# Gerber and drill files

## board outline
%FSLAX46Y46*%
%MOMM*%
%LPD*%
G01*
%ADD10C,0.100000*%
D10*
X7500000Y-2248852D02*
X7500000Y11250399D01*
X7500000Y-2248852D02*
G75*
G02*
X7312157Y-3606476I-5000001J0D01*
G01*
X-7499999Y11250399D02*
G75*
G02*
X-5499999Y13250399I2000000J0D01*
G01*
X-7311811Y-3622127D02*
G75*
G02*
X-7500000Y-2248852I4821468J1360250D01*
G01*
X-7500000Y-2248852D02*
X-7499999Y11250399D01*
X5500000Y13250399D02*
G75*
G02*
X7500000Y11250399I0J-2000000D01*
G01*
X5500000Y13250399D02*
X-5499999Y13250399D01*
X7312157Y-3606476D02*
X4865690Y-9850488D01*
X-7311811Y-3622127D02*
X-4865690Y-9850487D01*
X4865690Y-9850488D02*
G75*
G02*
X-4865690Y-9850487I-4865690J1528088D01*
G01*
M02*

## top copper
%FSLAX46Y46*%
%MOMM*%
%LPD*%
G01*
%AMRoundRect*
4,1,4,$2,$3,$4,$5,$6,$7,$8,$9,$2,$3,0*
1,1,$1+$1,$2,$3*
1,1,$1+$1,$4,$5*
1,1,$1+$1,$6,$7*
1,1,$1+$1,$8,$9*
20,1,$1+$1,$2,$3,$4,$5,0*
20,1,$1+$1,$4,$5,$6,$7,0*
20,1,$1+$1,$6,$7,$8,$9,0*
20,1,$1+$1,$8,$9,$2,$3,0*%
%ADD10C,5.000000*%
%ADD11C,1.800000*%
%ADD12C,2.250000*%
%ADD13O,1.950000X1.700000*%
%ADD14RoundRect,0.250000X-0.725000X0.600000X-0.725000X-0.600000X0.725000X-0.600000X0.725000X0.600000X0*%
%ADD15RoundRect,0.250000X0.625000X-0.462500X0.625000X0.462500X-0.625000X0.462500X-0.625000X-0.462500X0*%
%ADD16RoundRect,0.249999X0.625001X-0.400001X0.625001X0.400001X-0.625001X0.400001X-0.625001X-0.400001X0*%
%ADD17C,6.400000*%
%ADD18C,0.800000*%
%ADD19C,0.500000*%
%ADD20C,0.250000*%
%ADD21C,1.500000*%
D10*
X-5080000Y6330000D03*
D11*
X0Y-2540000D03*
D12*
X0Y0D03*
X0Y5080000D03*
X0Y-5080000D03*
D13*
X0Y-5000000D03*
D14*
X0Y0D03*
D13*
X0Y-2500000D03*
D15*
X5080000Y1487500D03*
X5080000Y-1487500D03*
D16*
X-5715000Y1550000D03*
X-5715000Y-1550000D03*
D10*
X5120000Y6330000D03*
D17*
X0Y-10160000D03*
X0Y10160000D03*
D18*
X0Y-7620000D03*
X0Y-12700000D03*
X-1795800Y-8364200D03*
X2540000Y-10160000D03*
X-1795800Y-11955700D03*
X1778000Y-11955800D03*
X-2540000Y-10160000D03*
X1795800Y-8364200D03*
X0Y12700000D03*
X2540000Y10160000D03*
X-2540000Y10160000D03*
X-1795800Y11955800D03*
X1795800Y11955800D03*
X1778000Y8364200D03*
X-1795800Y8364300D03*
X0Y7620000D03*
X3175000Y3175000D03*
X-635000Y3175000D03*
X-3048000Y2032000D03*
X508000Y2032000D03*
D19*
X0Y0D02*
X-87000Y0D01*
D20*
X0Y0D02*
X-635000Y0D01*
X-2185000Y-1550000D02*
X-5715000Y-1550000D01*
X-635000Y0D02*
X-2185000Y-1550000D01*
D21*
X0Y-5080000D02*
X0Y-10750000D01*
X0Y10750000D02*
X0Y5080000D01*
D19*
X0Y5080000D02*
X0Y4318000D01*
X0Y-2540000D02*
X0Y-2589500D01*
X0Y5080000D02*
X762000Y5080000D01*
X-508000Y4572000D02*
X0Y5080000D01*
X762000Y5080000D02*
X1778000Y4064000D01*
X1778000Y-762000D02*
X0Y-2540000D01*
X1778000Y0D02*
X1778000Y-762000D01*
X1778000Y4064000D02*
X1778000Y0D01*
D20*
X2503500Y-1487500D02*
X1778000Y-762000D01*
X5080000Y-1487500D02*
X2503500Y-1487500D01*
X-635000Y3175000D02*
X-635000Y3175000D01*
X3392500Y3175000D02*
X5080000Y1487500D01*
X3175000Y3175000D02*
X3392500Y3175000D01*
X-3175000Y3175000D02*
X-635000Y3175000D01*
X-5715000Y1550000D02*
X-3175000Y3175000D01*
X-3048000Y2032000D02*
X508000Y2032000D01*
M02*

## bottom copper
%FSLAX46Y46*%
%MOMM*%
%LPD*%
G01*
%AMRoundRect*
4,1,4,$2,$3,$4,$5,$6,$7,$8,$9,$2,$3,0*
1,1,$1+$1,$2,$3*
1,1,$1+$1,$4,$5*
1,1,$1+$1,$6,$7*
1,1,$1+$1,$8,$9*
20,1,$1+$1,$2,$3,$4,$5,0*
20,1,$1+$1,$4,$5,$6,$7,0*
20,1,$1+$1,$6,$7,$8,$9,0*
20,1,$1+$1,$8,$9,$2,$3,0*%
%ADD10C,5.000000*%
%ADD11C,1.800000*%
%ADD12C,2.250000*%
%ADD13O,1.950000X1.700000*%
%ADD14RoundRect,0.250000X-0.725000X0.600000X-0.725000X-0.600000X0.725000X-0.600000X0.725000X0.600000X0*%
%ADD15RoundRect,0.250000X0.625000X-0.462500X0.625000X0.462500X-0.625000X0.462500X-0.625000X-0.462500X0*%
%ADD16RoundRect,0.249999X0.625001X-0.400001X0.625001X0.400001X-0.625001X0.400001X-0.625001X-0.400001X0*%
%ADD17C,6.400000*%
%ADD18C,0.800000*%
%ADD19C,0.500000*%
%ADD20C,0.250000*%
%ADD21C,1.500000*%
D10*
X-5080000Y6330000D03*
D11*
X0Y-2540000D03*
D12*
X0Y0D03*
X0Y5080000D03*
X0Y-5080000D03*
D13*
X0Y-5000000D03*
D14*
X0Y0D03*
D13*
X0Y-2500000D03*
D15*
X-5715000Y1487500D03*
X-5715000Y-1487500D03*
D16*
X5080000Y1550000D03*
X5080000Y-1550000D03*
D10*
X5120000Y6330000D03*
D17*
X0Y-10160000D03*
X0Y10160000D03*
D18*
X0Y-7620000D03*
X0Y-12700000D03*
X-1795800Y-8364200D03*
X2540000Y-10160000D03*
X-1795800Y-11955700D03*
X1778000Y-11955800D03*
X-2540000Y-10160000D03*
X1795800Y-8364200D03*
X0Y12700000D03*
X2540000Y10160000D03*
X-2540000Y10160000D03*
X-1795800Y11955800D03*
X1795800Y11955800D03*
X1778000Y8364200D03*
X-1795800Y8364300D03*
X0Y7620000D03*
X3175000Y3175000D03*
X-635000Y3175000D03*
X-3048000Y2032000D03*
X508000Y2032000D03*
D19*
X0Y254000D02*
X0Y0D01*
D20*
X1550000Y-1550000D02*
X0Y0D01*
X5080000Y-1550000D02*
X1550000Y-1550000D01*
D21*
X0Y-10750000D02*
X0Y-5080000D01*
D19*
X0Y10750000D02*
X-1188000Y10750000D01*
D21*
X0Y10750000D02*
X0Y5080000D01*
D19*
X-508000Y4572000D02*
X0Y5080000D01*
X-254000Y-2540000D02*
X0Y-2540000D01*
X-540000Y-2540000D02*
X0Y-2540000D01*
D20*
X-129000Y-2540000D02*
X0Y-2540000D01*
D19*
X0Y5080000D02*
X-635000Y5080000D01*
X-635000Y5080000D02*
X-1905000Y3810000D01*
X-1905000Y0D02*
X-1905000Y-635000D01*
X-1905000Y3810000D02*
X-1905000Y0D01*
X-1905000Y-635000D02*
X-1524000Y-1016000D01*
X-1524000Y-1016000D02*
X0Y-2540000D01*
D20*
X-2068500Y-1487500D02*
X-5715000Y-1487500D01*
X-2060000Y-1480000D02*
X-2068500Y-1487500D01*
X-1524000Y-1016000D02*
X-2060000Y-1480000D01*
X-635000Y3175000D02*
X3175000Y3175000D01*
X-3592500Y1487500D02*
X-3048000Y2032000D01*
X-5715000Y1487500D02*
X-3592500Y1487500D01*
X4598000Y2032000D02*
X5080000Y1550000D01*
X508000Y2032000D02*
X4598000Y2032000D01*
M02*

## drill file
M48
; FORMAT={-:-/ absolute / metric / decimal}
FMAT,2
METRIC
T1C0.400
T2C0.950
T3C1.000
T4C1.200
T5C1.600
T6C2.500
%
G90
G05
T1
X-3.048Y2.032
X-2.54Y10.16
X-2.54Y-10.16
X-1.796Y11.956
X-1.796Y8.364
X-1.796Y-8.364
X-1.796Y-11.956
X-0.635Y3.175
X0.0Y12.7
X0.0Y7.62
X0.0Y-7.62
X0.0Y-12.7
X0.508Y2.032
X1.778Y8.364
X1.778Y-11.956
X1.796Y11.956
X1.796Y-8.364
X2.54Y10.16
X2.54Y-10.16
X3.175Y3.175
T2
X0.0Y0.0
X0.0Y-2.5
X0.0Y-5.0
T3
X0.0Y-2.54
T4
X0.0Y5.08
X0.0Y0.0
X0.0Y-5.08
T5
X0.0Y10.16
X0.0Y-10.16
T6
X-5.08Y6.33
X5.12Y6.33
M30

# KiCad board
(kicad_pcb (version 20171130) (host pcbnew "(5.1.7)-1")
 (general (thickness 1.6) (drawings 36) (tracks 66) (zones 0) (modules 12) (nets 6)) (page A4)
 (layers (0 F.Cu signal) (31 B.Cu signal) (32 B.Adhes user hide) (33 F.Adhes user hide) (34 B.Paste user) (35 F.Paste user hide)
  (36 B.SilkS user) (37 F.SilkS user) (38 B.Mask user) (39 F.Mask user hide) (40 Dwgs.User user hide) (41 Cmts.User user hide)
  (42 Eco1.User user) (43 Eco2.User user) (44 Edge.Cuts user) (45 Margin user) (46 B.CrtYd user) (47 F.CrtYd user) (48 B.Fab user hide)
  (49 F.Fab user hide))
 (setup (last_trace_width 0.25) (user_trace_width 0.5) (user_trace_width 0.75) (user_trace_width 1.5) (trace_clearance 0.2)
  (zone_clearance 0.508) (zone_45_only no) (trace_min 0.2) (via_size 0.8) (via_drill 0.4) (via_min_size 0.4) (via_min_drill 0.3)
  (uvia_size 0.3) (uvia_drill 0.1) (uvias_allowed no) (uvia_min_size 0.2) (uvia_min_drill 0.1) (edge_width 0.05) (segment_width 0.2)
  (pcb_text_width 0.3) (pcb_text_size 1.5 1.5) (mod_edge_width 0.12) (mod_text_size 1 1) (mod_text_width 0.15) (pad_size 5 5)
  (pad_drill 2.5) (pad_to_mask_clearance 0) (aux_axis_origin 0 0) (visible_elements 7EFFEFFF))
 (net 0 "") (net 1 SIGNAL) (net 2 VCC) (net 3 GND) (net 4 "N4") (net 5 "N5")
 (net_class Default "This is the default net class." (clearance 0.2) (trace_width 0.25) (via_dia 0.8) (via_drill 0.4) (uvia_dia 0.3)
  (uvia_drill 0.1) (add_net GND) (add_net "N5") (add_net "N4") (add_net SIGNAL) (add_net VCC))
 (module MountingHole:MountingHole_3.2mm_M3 (layer F.Cu) (at -5.08 -6.33)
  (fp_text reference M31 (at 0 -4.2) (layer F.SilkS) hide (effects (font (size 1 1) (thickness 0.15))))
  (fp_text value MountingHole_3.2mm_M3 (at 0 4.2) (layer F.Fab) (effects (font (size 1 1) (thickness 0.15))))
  (pad "" np_thru_hole circle (at 0 0) (size 5 5) (drill 2.5) (layers *.Cu *.Mask)))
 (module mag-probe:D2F (layer F.Cu) (at 0 0 270)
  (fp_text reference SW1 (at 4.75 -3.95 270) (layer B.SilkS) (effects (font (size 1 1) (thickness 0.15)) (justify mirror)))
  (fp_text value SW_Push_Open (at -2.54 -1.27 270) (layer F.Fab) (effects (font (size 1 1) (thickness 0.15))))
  (pad 4 thru_hole circle (at 2.54 0 270) (size 1.8 1.8) (drill 1) (layers *.Cu *.Mask) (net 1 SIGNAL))
  (pad 3 thru_hole circle (at 0 0 270) (size 2.25 2.25) (drill 1.2) (layers *.Cu *.Mask) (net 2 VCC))
  (pad 2 thru_hole circle (at -5.08 0 270) (size 2.25 2.25) (drill 1.2) (layers *.Cu *.Mask) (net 1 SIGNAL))
  (pad 1 thru_hole circle (at 5.08 0 270) (size 2.25 2.25) (drill 1.2) (layers *.Cu *.Mask) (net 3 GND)))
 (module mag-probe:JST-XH (layer F.Cu) (at 0 0 270)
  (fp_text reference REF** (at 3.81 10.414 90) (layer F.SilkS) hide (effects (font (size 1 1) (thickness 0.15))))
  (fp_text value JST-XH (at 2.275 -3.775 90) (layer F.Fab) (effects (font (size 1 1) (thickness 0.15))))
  (pad 3 thru_hole oval (at 5 0 270) (size 1.7 1.95) (drill 0.95) (layers *.Cu *.Mask) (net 3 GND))
  (pad 1 thru_hole roundrect (at 0 0 270) (size 1.7 1.95) (drill 0.95) (layers *.Cu *.Mask) (roundrect_rratio 0.1470588235294118))
  (pad 2 thru_hole oval (at 2.5 0 270) (size 1.7 1.95) (drill 0.95) (layers *.Cu *.Mask) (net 1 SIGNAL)))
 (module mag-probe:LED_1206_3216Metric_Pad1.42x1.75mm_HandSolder (layer B.Cu) (at -5.715 0 90)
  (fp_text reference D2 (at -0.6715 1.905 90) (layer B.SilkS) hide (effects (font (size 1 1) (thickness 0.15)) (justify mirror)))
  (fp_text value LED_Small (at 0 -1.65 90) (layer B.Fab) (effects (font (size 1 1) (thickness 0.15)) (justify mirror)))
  (pad 2 smd roundrect (at 1.4875 0 90) (size 1.425 1.75) (layers B.Cu B.Paste B.Mask) (roundrect_rratio 0.1754385964912281) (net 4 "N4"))
  (pad 1 smd roundrect (at -1.4875 0 90) (size 1.425 1.75) (layers B.Cu B.Paste B.Mask) (roundrect_rratio 0.1754385964912281) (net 1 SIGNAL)))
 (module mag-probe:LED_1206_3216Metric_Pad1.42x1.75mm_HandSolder (layer F.Cu) (at 5.08 0 90)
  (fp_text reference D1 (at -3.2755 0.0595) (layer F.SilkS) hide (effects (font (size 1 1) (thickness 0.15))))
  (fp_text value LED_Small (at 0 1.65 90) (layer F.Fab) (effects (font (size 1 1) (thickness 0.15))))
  (pad 2 smd roundrect (at 1.4875 0 90) (size 1.425 1.75) (layers F.Cu F.Paste F.Mask) (roundrect_rratio 0.1754385964912281) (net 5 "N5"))
  (pad 1 smd roundrect (at -1.4875 0 90) (size 1.425 1.75) (layers F.Cu F.Paste F.Mask) (roundrect_rratio 0.1754385964912281) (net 1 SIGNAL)))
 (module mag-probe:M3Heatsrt (layer F.Cu) (at -5.08 -6.33)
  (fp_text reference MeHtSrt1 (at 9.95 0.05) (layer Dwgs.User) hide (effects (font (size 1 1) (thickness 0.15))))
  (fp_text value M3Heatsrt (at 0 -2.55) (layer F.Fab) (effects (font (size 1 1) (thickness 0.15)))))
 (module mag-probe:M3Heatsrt (layer F.Cu) (at 5.08 -6.33)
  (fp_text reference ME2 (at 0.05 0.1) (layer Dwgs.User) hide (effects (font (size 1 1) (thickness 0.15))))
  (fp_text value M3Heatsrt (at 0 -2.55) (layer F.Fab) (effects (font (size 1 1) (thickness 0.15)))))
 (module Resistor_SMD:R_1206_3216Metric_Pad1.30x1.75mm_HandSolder (layer F.Cu) (at -5.715 0 90)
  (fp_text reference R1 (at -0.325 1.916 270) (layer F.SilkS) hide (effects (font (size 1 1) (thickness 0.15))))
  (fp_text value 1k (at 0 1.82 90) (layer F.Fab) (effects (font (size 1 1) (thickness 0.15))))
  (pad 2 smd roundrect (at 1.55 0 90) (size 1.3 1.75) (layers F.Cu F.Paste F.Mask) (roundrect_rratio 0.1923069230769231) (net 5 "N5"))
  (pad 1 smd roundrect (at -1.55 0 90) (size 1.3 1.75) (layers F.Cu F.Paste F.Mask) (roundrect_rratio 0.1923069230769231) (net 2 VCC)))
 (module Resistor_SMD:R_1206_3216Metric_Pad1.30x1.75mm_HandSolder (layer B.Cu) (at 5.08 0 90)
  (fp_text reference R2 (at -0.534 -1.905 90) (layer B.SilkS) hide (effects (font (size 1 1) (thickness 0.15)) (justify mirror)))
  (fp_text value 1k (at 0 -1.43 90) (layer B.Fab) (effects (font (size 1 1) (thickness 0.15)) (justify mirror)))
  (pad 2 smd roundrect (at 1.55 0 90) (size 1.3 1.75) (layers B.Cu B.Paste B.Mask) (roundrect_rratio 0.1923069230769231) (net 4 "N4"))
  (pad 1 smd roundrect (at -1.55 0 90) (size 1.3 1.75) (layers B.Cu B.Paste B.Mask) (roundrect_rratio 0.1923069230769231) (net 2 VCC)))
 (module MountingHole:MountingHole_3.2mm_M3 (layer F.Cu) (at 5.08 -6.33)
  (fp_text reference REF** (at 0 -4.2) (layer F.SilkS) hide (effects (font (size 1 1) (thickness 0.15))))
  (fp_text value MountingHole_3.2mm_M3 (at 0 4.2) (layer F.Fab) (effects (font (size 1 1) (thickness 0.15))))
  (pad "" np_thru_hole circle (at 0.04 0) (size 5 5) (drill 2.5) (layers *.Cu *.Mask)))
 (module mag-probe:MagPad (layer F.Cu) (at 0 10.16)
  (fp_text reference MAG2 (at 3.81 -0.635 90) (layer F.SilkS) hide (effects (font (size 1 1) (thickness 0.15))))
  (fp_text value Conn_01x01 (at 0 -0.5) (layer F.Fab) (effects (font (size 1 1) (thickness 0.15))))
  (pad 1 thru_hole circle (at 0 0) (size 6.4 6.4) (drill 1.6) (layers *.Cu *.Mask) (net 3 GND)))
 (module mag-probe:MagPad (layer F.Cu) (at 0 -10.16)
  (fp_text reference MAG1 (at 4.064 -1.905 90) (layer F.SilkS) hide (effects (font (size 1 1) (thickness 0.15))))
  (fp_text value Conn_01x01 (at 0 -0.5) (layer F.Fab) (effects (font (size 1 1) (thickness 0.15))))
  (pad 1 thru_hole circle (at 0 0) (size 6.4 6.4) (drill 1.6) (layers *.Cu *.Mask) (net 1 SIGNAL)))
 (gr_line (start 7.5 2.248852) (end 7.5 -11.250399) (layer Edge.Cuts) (width 0.1))
 (gr_arc (start 2.499999 2.248852) (end 7.312157 3.606476) (angle -15.75501346) (layer Edge.Cuts) (width 0.1))
 (gr_arc (start -5.499999 -11.250399) (end -5.499999 -13.250399) (angle -90) (layer Edge.Cuts) (width 0.1))
 (gr_arc (start -2.490343 2.261877) (end -7.5 2.248852) (angle -15.90398022) (layer Edge.Cuts) (width 0.1))
 (gr_line (start -7.5 2.248852) (end -7.499999 -11.250399) (layer Edge.Cuts) (width 0.1))
 (gr_arc (start 5.5 -11.250399) (end 7.5 -11.250399) (angle -90) (layer Edge.Cuts) (width 0.1))
 (gr_line (start 5.5 -13.250399) (end -5.499999 -13.250399) (layer Edge.Cuts) (width 0.1))
 (gr_line (start 7.312157 3.606476) (end 4.86569 9.850488) (layer Edge.Cuts) (width 0.1))
 (gr_line (start -7.311811 3.622127) (end -4.86569 9.850487) (layer Edge.Cuts) (width 0.1))
 (gr_arc (start 0 8.3224) (end -4.86569 9.850487) (angle -145.1298326) (layer Edge.Cuts) (width 0.1))
 (segment (start 0 -0.254) (end 0 0) (width 0.5) (layer B.Cu) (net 2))
 (segment (start 0 0) (end -0.087 0) (width 0.5) (layer F.Cu) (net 2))
 (segment (start 0 0) (end -0.635 0) (width 0.25) (layer F.Cu) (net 2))
 (segment (start -2.185 1.55) (end -5.715 1.55) (width 0.25) (layer F.Cu) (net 2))
 (segment (start -0.635 0) (end -2.185 1.55) (width 0.25) (layer F.Cu) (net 2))
 (segment (start 1.55 1.55) (end 0 0) (width 0.25) (layer B.Cu) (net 2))
 (segment (start 5.08 1.55) (end 1.55 1.55) (width 0.25) (layer B.Cu) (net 2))
 (segment (start 0 10.75) (end 0 5.08) (width 1.5) (layer B.Cu) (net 3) (status 30))
 (segment (start 0 5.08) (end 0 10.75) (width 1.5) (layer F.Cu) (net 3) (status 30))
 (via (at 0 7.62) (size 0.8) (drill 0.4) (layers F.Cu B.Cu) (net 3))
 (via (at 0 12.7) (size 0.8) (drill 0.4) (layers F.Cu B.Cu) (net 3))
 (via (at -1.7958 8.3642) (size 0.8) (drill 0.4) (layers F.Cu B.Cu) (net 3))
 (via (at 2.54 10.16) (size 0.8) (drill 0.4) (layers F.Cu B.Cu) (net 3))
 (via (at -1.7958 11.9557) (size 0.8) (drill 0.4) (layers F.Cu B.Cu) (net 3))
 (via (at 1.778 11.9558) (size 0.8) (drill 0.4) (layers F.Cu B.Cu) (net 3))
 (via (at -2.54 10.16) (size 0.8) (drill 0.4) (layers F.Cu B.Cu) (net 3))
 (via (at 1.7958 8.3642) (size 0.8) (drill 0.4) (layers F.Cu B.Cu) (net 3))
 (via (at 0 -12.7) (size 0.8) (drill 0.4) (layers F.Cu B.Cu) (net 1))
 (via (at 2.54 -10.16) (size 0.8) (drill 0.4) (layers F.Cu B.Cu) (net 1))
 (via (at -2.54 -10.16) (size 0.8) (drill 0.4) (layers F.Cu B.Cu) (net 1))
 (via (at -1.7958 -11.9558) (size 0.8) (drill 0.4) (layers F.Cu B.Cu) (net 1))
 (via (at 1.7958 -11.9558) (size 0.8) (drill 0.4) (layers F.Cu B.Cu) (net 1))
 (via (at 1.778 -8.3642) (size 0.8) (drill 0.4) (layers F.Cu B.Cu) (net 1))
 (via (at -1.7958 -8.3643) (size 0.8) (drill 0.4) (layers F.Cu B.Cu) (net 1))
 (via (at 0 -7.62) (size 0.8) (drill 0.4) (layers F.Cu B.Cu) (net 1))
 (segment (start 0 -10.75) (end -1.188 -10.75) (width 0.5) (layer B.Cu) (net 1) (status 30))
 (segment (start 0 -10.75) (end 0 -5.08) (width 1.5) (layer B.Cu) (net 1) (status 30))
 (segment (start -0.508 -4.572) (end 0 -5.08) (width 0.5) (layer B.Cu) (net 1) (status 30))
 (segment (start 0 -10.75) (end 0 -5.08) (width 1.5) (layer F.Cu) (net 1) (status 30))
 (segment (start -0.254 2.54) (end 0 2.54) (width 0.5) (layer B.Cu) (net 1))
 (segment (start 0 -5.08) (end 0 -4.318) (width 0.5) (layer F.Cu) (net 1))
 (segment (start 0 2.54) (end 0 2.5895) (width 0.5) (layer F.Cu) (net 1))
 (segment (start -0.54 2.54) (end 0 2.54) (width 0.5) (layer B.Cu) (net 1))
 (segment (start -0.129 2.54) (end 0 2.54) (width 0.25) (layer B.Cu) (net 1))
 (segment (start 0 -5.08) (end 0.762 -5.08) (width 0.5) (layer F.Cu) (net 1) (status 30))
 (segment (start -0.508 -4.572) (end 0 -5.08) (width 0.5) (layer F.Cu) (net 1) (status 30))
 (segment (start 0 -5.08) (end -0.635 -5.08) (width 0.5) (layer B.Cu) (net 1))
 (segment (start -0.635 -5.08) (end -1.905 -3.81) (width 0.5) (layer B.Cu) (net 1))
 (segment (start 0.762 -5.08) (end 1.778 -4.064) (width 0.5) (layer F.Cu) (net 1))
 (segment (start 1.778 0.762) (end 0 2.54) (width 0.5) (layer F.Cu) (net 1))
 (segment (start 1.778 0) (end 1.778 0.762) (width 0.5) (layer F.Cu) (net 1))
 (segment (start 1.778 -4.064) (end 1.778 0) (width 0.5) (layer F.Cu) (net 1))
 (segment (start -1.905 0) (end -1.905 0.635) (width 0.5) (layer B.Cu) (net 1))
 (segment (start -1.905 -3.81) (end -1.905 0) (width 0.5) (layer B.Cu) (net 1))
 (segment (start 2.5035 1.4875) (end 1.778 0.762) (width 0.25) (layer F.Cu) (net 1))
 (segment (start 5.08 1.4875) (end 2.5035 1.4875) (width 0.25) (layer F.Cu) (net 1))
 (segment (start -1.905 0.635) (end -1.524 1.016) (width 0.5) (layer B.Cu) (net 1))
 (segment (start -1.524 1.016) (end 0 2.54) (width 0.5) (layer B.Cu) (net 1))
 (segment (start -2.0685 1.4875) (end -5.715 1.4875) (width 0.25) (layer B.Cu) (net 1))
 (segment (start -2.06 1.48) (end -2.0685 1.4875) (width 0.25) (layer B.Cu) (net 1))
 (segment (start -1.524 1.016) (end -2.06 1.48) (width 0.25) (layer B.Cu) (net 1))
 (via (at 3.175 -3.175) (size 0.8) (drill 0.4) (layers F.Cu B.Cu) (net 5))
 (segment (start -0.635 -3.175) (end -0.635 -3.175) (width 0.25) (layer F.Cu) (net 5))
 (via (at -0.635 -3.175) (size 0.8) (drill 0.4) (layers F.Cu B.Cu) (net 5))
 (segment (start -0.635 -3.175) (end 3.175 -3.175) (width 0.25) (layer B.Cu) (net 5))
 (segment (start 3.3925 -3.175) (end 5.08 -1.4875) (width 0.25) (layer F.Cu) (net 5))
 (segment (start 3.175 -3.175) (end 3.3925 -3.175) (width 0.25) (layer F.Cu) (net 5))
 (segment (start -3.175 -3.175) (end -0.635 -3.175) (width 0.25) (layer F.Cu) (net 5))
 (segment (start -5.715 -1.55) (end -3.175 -3.175) (width 0.25) (layer F.Cu) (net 5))
 (via (at -3.048 -2.032) (size 0.8) (drill 0.4) (layers F.Cu B.Cu) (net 4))
 (via (at 0.508 -2.032) (size 0.8) (drill 0.4) (layers F.Cu B.Cu) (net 4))
 (segment (start -3.5925 -1.4875) (end -3.048 -2.032) (width 0.25) (layer B.Cu) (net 4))
 (segment (start -5.715 -1.4875) (end -3.5925 -1.4875) (width 0.25) (layer B.Cu) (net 4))
 (segment (start 4.598 -2.032) (end 5.08 -1.55) (width 0.25) (layer B.Cu) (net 4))
 (segment (start 0.508 -2.032) (end 4.598 -2.032) (width 0.25) (layer B.Cu) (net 4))
 (segment (start -3.048 -2.032) (end 0.508 -2.032) (width 0.25) (layer F.Cu) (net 4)))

